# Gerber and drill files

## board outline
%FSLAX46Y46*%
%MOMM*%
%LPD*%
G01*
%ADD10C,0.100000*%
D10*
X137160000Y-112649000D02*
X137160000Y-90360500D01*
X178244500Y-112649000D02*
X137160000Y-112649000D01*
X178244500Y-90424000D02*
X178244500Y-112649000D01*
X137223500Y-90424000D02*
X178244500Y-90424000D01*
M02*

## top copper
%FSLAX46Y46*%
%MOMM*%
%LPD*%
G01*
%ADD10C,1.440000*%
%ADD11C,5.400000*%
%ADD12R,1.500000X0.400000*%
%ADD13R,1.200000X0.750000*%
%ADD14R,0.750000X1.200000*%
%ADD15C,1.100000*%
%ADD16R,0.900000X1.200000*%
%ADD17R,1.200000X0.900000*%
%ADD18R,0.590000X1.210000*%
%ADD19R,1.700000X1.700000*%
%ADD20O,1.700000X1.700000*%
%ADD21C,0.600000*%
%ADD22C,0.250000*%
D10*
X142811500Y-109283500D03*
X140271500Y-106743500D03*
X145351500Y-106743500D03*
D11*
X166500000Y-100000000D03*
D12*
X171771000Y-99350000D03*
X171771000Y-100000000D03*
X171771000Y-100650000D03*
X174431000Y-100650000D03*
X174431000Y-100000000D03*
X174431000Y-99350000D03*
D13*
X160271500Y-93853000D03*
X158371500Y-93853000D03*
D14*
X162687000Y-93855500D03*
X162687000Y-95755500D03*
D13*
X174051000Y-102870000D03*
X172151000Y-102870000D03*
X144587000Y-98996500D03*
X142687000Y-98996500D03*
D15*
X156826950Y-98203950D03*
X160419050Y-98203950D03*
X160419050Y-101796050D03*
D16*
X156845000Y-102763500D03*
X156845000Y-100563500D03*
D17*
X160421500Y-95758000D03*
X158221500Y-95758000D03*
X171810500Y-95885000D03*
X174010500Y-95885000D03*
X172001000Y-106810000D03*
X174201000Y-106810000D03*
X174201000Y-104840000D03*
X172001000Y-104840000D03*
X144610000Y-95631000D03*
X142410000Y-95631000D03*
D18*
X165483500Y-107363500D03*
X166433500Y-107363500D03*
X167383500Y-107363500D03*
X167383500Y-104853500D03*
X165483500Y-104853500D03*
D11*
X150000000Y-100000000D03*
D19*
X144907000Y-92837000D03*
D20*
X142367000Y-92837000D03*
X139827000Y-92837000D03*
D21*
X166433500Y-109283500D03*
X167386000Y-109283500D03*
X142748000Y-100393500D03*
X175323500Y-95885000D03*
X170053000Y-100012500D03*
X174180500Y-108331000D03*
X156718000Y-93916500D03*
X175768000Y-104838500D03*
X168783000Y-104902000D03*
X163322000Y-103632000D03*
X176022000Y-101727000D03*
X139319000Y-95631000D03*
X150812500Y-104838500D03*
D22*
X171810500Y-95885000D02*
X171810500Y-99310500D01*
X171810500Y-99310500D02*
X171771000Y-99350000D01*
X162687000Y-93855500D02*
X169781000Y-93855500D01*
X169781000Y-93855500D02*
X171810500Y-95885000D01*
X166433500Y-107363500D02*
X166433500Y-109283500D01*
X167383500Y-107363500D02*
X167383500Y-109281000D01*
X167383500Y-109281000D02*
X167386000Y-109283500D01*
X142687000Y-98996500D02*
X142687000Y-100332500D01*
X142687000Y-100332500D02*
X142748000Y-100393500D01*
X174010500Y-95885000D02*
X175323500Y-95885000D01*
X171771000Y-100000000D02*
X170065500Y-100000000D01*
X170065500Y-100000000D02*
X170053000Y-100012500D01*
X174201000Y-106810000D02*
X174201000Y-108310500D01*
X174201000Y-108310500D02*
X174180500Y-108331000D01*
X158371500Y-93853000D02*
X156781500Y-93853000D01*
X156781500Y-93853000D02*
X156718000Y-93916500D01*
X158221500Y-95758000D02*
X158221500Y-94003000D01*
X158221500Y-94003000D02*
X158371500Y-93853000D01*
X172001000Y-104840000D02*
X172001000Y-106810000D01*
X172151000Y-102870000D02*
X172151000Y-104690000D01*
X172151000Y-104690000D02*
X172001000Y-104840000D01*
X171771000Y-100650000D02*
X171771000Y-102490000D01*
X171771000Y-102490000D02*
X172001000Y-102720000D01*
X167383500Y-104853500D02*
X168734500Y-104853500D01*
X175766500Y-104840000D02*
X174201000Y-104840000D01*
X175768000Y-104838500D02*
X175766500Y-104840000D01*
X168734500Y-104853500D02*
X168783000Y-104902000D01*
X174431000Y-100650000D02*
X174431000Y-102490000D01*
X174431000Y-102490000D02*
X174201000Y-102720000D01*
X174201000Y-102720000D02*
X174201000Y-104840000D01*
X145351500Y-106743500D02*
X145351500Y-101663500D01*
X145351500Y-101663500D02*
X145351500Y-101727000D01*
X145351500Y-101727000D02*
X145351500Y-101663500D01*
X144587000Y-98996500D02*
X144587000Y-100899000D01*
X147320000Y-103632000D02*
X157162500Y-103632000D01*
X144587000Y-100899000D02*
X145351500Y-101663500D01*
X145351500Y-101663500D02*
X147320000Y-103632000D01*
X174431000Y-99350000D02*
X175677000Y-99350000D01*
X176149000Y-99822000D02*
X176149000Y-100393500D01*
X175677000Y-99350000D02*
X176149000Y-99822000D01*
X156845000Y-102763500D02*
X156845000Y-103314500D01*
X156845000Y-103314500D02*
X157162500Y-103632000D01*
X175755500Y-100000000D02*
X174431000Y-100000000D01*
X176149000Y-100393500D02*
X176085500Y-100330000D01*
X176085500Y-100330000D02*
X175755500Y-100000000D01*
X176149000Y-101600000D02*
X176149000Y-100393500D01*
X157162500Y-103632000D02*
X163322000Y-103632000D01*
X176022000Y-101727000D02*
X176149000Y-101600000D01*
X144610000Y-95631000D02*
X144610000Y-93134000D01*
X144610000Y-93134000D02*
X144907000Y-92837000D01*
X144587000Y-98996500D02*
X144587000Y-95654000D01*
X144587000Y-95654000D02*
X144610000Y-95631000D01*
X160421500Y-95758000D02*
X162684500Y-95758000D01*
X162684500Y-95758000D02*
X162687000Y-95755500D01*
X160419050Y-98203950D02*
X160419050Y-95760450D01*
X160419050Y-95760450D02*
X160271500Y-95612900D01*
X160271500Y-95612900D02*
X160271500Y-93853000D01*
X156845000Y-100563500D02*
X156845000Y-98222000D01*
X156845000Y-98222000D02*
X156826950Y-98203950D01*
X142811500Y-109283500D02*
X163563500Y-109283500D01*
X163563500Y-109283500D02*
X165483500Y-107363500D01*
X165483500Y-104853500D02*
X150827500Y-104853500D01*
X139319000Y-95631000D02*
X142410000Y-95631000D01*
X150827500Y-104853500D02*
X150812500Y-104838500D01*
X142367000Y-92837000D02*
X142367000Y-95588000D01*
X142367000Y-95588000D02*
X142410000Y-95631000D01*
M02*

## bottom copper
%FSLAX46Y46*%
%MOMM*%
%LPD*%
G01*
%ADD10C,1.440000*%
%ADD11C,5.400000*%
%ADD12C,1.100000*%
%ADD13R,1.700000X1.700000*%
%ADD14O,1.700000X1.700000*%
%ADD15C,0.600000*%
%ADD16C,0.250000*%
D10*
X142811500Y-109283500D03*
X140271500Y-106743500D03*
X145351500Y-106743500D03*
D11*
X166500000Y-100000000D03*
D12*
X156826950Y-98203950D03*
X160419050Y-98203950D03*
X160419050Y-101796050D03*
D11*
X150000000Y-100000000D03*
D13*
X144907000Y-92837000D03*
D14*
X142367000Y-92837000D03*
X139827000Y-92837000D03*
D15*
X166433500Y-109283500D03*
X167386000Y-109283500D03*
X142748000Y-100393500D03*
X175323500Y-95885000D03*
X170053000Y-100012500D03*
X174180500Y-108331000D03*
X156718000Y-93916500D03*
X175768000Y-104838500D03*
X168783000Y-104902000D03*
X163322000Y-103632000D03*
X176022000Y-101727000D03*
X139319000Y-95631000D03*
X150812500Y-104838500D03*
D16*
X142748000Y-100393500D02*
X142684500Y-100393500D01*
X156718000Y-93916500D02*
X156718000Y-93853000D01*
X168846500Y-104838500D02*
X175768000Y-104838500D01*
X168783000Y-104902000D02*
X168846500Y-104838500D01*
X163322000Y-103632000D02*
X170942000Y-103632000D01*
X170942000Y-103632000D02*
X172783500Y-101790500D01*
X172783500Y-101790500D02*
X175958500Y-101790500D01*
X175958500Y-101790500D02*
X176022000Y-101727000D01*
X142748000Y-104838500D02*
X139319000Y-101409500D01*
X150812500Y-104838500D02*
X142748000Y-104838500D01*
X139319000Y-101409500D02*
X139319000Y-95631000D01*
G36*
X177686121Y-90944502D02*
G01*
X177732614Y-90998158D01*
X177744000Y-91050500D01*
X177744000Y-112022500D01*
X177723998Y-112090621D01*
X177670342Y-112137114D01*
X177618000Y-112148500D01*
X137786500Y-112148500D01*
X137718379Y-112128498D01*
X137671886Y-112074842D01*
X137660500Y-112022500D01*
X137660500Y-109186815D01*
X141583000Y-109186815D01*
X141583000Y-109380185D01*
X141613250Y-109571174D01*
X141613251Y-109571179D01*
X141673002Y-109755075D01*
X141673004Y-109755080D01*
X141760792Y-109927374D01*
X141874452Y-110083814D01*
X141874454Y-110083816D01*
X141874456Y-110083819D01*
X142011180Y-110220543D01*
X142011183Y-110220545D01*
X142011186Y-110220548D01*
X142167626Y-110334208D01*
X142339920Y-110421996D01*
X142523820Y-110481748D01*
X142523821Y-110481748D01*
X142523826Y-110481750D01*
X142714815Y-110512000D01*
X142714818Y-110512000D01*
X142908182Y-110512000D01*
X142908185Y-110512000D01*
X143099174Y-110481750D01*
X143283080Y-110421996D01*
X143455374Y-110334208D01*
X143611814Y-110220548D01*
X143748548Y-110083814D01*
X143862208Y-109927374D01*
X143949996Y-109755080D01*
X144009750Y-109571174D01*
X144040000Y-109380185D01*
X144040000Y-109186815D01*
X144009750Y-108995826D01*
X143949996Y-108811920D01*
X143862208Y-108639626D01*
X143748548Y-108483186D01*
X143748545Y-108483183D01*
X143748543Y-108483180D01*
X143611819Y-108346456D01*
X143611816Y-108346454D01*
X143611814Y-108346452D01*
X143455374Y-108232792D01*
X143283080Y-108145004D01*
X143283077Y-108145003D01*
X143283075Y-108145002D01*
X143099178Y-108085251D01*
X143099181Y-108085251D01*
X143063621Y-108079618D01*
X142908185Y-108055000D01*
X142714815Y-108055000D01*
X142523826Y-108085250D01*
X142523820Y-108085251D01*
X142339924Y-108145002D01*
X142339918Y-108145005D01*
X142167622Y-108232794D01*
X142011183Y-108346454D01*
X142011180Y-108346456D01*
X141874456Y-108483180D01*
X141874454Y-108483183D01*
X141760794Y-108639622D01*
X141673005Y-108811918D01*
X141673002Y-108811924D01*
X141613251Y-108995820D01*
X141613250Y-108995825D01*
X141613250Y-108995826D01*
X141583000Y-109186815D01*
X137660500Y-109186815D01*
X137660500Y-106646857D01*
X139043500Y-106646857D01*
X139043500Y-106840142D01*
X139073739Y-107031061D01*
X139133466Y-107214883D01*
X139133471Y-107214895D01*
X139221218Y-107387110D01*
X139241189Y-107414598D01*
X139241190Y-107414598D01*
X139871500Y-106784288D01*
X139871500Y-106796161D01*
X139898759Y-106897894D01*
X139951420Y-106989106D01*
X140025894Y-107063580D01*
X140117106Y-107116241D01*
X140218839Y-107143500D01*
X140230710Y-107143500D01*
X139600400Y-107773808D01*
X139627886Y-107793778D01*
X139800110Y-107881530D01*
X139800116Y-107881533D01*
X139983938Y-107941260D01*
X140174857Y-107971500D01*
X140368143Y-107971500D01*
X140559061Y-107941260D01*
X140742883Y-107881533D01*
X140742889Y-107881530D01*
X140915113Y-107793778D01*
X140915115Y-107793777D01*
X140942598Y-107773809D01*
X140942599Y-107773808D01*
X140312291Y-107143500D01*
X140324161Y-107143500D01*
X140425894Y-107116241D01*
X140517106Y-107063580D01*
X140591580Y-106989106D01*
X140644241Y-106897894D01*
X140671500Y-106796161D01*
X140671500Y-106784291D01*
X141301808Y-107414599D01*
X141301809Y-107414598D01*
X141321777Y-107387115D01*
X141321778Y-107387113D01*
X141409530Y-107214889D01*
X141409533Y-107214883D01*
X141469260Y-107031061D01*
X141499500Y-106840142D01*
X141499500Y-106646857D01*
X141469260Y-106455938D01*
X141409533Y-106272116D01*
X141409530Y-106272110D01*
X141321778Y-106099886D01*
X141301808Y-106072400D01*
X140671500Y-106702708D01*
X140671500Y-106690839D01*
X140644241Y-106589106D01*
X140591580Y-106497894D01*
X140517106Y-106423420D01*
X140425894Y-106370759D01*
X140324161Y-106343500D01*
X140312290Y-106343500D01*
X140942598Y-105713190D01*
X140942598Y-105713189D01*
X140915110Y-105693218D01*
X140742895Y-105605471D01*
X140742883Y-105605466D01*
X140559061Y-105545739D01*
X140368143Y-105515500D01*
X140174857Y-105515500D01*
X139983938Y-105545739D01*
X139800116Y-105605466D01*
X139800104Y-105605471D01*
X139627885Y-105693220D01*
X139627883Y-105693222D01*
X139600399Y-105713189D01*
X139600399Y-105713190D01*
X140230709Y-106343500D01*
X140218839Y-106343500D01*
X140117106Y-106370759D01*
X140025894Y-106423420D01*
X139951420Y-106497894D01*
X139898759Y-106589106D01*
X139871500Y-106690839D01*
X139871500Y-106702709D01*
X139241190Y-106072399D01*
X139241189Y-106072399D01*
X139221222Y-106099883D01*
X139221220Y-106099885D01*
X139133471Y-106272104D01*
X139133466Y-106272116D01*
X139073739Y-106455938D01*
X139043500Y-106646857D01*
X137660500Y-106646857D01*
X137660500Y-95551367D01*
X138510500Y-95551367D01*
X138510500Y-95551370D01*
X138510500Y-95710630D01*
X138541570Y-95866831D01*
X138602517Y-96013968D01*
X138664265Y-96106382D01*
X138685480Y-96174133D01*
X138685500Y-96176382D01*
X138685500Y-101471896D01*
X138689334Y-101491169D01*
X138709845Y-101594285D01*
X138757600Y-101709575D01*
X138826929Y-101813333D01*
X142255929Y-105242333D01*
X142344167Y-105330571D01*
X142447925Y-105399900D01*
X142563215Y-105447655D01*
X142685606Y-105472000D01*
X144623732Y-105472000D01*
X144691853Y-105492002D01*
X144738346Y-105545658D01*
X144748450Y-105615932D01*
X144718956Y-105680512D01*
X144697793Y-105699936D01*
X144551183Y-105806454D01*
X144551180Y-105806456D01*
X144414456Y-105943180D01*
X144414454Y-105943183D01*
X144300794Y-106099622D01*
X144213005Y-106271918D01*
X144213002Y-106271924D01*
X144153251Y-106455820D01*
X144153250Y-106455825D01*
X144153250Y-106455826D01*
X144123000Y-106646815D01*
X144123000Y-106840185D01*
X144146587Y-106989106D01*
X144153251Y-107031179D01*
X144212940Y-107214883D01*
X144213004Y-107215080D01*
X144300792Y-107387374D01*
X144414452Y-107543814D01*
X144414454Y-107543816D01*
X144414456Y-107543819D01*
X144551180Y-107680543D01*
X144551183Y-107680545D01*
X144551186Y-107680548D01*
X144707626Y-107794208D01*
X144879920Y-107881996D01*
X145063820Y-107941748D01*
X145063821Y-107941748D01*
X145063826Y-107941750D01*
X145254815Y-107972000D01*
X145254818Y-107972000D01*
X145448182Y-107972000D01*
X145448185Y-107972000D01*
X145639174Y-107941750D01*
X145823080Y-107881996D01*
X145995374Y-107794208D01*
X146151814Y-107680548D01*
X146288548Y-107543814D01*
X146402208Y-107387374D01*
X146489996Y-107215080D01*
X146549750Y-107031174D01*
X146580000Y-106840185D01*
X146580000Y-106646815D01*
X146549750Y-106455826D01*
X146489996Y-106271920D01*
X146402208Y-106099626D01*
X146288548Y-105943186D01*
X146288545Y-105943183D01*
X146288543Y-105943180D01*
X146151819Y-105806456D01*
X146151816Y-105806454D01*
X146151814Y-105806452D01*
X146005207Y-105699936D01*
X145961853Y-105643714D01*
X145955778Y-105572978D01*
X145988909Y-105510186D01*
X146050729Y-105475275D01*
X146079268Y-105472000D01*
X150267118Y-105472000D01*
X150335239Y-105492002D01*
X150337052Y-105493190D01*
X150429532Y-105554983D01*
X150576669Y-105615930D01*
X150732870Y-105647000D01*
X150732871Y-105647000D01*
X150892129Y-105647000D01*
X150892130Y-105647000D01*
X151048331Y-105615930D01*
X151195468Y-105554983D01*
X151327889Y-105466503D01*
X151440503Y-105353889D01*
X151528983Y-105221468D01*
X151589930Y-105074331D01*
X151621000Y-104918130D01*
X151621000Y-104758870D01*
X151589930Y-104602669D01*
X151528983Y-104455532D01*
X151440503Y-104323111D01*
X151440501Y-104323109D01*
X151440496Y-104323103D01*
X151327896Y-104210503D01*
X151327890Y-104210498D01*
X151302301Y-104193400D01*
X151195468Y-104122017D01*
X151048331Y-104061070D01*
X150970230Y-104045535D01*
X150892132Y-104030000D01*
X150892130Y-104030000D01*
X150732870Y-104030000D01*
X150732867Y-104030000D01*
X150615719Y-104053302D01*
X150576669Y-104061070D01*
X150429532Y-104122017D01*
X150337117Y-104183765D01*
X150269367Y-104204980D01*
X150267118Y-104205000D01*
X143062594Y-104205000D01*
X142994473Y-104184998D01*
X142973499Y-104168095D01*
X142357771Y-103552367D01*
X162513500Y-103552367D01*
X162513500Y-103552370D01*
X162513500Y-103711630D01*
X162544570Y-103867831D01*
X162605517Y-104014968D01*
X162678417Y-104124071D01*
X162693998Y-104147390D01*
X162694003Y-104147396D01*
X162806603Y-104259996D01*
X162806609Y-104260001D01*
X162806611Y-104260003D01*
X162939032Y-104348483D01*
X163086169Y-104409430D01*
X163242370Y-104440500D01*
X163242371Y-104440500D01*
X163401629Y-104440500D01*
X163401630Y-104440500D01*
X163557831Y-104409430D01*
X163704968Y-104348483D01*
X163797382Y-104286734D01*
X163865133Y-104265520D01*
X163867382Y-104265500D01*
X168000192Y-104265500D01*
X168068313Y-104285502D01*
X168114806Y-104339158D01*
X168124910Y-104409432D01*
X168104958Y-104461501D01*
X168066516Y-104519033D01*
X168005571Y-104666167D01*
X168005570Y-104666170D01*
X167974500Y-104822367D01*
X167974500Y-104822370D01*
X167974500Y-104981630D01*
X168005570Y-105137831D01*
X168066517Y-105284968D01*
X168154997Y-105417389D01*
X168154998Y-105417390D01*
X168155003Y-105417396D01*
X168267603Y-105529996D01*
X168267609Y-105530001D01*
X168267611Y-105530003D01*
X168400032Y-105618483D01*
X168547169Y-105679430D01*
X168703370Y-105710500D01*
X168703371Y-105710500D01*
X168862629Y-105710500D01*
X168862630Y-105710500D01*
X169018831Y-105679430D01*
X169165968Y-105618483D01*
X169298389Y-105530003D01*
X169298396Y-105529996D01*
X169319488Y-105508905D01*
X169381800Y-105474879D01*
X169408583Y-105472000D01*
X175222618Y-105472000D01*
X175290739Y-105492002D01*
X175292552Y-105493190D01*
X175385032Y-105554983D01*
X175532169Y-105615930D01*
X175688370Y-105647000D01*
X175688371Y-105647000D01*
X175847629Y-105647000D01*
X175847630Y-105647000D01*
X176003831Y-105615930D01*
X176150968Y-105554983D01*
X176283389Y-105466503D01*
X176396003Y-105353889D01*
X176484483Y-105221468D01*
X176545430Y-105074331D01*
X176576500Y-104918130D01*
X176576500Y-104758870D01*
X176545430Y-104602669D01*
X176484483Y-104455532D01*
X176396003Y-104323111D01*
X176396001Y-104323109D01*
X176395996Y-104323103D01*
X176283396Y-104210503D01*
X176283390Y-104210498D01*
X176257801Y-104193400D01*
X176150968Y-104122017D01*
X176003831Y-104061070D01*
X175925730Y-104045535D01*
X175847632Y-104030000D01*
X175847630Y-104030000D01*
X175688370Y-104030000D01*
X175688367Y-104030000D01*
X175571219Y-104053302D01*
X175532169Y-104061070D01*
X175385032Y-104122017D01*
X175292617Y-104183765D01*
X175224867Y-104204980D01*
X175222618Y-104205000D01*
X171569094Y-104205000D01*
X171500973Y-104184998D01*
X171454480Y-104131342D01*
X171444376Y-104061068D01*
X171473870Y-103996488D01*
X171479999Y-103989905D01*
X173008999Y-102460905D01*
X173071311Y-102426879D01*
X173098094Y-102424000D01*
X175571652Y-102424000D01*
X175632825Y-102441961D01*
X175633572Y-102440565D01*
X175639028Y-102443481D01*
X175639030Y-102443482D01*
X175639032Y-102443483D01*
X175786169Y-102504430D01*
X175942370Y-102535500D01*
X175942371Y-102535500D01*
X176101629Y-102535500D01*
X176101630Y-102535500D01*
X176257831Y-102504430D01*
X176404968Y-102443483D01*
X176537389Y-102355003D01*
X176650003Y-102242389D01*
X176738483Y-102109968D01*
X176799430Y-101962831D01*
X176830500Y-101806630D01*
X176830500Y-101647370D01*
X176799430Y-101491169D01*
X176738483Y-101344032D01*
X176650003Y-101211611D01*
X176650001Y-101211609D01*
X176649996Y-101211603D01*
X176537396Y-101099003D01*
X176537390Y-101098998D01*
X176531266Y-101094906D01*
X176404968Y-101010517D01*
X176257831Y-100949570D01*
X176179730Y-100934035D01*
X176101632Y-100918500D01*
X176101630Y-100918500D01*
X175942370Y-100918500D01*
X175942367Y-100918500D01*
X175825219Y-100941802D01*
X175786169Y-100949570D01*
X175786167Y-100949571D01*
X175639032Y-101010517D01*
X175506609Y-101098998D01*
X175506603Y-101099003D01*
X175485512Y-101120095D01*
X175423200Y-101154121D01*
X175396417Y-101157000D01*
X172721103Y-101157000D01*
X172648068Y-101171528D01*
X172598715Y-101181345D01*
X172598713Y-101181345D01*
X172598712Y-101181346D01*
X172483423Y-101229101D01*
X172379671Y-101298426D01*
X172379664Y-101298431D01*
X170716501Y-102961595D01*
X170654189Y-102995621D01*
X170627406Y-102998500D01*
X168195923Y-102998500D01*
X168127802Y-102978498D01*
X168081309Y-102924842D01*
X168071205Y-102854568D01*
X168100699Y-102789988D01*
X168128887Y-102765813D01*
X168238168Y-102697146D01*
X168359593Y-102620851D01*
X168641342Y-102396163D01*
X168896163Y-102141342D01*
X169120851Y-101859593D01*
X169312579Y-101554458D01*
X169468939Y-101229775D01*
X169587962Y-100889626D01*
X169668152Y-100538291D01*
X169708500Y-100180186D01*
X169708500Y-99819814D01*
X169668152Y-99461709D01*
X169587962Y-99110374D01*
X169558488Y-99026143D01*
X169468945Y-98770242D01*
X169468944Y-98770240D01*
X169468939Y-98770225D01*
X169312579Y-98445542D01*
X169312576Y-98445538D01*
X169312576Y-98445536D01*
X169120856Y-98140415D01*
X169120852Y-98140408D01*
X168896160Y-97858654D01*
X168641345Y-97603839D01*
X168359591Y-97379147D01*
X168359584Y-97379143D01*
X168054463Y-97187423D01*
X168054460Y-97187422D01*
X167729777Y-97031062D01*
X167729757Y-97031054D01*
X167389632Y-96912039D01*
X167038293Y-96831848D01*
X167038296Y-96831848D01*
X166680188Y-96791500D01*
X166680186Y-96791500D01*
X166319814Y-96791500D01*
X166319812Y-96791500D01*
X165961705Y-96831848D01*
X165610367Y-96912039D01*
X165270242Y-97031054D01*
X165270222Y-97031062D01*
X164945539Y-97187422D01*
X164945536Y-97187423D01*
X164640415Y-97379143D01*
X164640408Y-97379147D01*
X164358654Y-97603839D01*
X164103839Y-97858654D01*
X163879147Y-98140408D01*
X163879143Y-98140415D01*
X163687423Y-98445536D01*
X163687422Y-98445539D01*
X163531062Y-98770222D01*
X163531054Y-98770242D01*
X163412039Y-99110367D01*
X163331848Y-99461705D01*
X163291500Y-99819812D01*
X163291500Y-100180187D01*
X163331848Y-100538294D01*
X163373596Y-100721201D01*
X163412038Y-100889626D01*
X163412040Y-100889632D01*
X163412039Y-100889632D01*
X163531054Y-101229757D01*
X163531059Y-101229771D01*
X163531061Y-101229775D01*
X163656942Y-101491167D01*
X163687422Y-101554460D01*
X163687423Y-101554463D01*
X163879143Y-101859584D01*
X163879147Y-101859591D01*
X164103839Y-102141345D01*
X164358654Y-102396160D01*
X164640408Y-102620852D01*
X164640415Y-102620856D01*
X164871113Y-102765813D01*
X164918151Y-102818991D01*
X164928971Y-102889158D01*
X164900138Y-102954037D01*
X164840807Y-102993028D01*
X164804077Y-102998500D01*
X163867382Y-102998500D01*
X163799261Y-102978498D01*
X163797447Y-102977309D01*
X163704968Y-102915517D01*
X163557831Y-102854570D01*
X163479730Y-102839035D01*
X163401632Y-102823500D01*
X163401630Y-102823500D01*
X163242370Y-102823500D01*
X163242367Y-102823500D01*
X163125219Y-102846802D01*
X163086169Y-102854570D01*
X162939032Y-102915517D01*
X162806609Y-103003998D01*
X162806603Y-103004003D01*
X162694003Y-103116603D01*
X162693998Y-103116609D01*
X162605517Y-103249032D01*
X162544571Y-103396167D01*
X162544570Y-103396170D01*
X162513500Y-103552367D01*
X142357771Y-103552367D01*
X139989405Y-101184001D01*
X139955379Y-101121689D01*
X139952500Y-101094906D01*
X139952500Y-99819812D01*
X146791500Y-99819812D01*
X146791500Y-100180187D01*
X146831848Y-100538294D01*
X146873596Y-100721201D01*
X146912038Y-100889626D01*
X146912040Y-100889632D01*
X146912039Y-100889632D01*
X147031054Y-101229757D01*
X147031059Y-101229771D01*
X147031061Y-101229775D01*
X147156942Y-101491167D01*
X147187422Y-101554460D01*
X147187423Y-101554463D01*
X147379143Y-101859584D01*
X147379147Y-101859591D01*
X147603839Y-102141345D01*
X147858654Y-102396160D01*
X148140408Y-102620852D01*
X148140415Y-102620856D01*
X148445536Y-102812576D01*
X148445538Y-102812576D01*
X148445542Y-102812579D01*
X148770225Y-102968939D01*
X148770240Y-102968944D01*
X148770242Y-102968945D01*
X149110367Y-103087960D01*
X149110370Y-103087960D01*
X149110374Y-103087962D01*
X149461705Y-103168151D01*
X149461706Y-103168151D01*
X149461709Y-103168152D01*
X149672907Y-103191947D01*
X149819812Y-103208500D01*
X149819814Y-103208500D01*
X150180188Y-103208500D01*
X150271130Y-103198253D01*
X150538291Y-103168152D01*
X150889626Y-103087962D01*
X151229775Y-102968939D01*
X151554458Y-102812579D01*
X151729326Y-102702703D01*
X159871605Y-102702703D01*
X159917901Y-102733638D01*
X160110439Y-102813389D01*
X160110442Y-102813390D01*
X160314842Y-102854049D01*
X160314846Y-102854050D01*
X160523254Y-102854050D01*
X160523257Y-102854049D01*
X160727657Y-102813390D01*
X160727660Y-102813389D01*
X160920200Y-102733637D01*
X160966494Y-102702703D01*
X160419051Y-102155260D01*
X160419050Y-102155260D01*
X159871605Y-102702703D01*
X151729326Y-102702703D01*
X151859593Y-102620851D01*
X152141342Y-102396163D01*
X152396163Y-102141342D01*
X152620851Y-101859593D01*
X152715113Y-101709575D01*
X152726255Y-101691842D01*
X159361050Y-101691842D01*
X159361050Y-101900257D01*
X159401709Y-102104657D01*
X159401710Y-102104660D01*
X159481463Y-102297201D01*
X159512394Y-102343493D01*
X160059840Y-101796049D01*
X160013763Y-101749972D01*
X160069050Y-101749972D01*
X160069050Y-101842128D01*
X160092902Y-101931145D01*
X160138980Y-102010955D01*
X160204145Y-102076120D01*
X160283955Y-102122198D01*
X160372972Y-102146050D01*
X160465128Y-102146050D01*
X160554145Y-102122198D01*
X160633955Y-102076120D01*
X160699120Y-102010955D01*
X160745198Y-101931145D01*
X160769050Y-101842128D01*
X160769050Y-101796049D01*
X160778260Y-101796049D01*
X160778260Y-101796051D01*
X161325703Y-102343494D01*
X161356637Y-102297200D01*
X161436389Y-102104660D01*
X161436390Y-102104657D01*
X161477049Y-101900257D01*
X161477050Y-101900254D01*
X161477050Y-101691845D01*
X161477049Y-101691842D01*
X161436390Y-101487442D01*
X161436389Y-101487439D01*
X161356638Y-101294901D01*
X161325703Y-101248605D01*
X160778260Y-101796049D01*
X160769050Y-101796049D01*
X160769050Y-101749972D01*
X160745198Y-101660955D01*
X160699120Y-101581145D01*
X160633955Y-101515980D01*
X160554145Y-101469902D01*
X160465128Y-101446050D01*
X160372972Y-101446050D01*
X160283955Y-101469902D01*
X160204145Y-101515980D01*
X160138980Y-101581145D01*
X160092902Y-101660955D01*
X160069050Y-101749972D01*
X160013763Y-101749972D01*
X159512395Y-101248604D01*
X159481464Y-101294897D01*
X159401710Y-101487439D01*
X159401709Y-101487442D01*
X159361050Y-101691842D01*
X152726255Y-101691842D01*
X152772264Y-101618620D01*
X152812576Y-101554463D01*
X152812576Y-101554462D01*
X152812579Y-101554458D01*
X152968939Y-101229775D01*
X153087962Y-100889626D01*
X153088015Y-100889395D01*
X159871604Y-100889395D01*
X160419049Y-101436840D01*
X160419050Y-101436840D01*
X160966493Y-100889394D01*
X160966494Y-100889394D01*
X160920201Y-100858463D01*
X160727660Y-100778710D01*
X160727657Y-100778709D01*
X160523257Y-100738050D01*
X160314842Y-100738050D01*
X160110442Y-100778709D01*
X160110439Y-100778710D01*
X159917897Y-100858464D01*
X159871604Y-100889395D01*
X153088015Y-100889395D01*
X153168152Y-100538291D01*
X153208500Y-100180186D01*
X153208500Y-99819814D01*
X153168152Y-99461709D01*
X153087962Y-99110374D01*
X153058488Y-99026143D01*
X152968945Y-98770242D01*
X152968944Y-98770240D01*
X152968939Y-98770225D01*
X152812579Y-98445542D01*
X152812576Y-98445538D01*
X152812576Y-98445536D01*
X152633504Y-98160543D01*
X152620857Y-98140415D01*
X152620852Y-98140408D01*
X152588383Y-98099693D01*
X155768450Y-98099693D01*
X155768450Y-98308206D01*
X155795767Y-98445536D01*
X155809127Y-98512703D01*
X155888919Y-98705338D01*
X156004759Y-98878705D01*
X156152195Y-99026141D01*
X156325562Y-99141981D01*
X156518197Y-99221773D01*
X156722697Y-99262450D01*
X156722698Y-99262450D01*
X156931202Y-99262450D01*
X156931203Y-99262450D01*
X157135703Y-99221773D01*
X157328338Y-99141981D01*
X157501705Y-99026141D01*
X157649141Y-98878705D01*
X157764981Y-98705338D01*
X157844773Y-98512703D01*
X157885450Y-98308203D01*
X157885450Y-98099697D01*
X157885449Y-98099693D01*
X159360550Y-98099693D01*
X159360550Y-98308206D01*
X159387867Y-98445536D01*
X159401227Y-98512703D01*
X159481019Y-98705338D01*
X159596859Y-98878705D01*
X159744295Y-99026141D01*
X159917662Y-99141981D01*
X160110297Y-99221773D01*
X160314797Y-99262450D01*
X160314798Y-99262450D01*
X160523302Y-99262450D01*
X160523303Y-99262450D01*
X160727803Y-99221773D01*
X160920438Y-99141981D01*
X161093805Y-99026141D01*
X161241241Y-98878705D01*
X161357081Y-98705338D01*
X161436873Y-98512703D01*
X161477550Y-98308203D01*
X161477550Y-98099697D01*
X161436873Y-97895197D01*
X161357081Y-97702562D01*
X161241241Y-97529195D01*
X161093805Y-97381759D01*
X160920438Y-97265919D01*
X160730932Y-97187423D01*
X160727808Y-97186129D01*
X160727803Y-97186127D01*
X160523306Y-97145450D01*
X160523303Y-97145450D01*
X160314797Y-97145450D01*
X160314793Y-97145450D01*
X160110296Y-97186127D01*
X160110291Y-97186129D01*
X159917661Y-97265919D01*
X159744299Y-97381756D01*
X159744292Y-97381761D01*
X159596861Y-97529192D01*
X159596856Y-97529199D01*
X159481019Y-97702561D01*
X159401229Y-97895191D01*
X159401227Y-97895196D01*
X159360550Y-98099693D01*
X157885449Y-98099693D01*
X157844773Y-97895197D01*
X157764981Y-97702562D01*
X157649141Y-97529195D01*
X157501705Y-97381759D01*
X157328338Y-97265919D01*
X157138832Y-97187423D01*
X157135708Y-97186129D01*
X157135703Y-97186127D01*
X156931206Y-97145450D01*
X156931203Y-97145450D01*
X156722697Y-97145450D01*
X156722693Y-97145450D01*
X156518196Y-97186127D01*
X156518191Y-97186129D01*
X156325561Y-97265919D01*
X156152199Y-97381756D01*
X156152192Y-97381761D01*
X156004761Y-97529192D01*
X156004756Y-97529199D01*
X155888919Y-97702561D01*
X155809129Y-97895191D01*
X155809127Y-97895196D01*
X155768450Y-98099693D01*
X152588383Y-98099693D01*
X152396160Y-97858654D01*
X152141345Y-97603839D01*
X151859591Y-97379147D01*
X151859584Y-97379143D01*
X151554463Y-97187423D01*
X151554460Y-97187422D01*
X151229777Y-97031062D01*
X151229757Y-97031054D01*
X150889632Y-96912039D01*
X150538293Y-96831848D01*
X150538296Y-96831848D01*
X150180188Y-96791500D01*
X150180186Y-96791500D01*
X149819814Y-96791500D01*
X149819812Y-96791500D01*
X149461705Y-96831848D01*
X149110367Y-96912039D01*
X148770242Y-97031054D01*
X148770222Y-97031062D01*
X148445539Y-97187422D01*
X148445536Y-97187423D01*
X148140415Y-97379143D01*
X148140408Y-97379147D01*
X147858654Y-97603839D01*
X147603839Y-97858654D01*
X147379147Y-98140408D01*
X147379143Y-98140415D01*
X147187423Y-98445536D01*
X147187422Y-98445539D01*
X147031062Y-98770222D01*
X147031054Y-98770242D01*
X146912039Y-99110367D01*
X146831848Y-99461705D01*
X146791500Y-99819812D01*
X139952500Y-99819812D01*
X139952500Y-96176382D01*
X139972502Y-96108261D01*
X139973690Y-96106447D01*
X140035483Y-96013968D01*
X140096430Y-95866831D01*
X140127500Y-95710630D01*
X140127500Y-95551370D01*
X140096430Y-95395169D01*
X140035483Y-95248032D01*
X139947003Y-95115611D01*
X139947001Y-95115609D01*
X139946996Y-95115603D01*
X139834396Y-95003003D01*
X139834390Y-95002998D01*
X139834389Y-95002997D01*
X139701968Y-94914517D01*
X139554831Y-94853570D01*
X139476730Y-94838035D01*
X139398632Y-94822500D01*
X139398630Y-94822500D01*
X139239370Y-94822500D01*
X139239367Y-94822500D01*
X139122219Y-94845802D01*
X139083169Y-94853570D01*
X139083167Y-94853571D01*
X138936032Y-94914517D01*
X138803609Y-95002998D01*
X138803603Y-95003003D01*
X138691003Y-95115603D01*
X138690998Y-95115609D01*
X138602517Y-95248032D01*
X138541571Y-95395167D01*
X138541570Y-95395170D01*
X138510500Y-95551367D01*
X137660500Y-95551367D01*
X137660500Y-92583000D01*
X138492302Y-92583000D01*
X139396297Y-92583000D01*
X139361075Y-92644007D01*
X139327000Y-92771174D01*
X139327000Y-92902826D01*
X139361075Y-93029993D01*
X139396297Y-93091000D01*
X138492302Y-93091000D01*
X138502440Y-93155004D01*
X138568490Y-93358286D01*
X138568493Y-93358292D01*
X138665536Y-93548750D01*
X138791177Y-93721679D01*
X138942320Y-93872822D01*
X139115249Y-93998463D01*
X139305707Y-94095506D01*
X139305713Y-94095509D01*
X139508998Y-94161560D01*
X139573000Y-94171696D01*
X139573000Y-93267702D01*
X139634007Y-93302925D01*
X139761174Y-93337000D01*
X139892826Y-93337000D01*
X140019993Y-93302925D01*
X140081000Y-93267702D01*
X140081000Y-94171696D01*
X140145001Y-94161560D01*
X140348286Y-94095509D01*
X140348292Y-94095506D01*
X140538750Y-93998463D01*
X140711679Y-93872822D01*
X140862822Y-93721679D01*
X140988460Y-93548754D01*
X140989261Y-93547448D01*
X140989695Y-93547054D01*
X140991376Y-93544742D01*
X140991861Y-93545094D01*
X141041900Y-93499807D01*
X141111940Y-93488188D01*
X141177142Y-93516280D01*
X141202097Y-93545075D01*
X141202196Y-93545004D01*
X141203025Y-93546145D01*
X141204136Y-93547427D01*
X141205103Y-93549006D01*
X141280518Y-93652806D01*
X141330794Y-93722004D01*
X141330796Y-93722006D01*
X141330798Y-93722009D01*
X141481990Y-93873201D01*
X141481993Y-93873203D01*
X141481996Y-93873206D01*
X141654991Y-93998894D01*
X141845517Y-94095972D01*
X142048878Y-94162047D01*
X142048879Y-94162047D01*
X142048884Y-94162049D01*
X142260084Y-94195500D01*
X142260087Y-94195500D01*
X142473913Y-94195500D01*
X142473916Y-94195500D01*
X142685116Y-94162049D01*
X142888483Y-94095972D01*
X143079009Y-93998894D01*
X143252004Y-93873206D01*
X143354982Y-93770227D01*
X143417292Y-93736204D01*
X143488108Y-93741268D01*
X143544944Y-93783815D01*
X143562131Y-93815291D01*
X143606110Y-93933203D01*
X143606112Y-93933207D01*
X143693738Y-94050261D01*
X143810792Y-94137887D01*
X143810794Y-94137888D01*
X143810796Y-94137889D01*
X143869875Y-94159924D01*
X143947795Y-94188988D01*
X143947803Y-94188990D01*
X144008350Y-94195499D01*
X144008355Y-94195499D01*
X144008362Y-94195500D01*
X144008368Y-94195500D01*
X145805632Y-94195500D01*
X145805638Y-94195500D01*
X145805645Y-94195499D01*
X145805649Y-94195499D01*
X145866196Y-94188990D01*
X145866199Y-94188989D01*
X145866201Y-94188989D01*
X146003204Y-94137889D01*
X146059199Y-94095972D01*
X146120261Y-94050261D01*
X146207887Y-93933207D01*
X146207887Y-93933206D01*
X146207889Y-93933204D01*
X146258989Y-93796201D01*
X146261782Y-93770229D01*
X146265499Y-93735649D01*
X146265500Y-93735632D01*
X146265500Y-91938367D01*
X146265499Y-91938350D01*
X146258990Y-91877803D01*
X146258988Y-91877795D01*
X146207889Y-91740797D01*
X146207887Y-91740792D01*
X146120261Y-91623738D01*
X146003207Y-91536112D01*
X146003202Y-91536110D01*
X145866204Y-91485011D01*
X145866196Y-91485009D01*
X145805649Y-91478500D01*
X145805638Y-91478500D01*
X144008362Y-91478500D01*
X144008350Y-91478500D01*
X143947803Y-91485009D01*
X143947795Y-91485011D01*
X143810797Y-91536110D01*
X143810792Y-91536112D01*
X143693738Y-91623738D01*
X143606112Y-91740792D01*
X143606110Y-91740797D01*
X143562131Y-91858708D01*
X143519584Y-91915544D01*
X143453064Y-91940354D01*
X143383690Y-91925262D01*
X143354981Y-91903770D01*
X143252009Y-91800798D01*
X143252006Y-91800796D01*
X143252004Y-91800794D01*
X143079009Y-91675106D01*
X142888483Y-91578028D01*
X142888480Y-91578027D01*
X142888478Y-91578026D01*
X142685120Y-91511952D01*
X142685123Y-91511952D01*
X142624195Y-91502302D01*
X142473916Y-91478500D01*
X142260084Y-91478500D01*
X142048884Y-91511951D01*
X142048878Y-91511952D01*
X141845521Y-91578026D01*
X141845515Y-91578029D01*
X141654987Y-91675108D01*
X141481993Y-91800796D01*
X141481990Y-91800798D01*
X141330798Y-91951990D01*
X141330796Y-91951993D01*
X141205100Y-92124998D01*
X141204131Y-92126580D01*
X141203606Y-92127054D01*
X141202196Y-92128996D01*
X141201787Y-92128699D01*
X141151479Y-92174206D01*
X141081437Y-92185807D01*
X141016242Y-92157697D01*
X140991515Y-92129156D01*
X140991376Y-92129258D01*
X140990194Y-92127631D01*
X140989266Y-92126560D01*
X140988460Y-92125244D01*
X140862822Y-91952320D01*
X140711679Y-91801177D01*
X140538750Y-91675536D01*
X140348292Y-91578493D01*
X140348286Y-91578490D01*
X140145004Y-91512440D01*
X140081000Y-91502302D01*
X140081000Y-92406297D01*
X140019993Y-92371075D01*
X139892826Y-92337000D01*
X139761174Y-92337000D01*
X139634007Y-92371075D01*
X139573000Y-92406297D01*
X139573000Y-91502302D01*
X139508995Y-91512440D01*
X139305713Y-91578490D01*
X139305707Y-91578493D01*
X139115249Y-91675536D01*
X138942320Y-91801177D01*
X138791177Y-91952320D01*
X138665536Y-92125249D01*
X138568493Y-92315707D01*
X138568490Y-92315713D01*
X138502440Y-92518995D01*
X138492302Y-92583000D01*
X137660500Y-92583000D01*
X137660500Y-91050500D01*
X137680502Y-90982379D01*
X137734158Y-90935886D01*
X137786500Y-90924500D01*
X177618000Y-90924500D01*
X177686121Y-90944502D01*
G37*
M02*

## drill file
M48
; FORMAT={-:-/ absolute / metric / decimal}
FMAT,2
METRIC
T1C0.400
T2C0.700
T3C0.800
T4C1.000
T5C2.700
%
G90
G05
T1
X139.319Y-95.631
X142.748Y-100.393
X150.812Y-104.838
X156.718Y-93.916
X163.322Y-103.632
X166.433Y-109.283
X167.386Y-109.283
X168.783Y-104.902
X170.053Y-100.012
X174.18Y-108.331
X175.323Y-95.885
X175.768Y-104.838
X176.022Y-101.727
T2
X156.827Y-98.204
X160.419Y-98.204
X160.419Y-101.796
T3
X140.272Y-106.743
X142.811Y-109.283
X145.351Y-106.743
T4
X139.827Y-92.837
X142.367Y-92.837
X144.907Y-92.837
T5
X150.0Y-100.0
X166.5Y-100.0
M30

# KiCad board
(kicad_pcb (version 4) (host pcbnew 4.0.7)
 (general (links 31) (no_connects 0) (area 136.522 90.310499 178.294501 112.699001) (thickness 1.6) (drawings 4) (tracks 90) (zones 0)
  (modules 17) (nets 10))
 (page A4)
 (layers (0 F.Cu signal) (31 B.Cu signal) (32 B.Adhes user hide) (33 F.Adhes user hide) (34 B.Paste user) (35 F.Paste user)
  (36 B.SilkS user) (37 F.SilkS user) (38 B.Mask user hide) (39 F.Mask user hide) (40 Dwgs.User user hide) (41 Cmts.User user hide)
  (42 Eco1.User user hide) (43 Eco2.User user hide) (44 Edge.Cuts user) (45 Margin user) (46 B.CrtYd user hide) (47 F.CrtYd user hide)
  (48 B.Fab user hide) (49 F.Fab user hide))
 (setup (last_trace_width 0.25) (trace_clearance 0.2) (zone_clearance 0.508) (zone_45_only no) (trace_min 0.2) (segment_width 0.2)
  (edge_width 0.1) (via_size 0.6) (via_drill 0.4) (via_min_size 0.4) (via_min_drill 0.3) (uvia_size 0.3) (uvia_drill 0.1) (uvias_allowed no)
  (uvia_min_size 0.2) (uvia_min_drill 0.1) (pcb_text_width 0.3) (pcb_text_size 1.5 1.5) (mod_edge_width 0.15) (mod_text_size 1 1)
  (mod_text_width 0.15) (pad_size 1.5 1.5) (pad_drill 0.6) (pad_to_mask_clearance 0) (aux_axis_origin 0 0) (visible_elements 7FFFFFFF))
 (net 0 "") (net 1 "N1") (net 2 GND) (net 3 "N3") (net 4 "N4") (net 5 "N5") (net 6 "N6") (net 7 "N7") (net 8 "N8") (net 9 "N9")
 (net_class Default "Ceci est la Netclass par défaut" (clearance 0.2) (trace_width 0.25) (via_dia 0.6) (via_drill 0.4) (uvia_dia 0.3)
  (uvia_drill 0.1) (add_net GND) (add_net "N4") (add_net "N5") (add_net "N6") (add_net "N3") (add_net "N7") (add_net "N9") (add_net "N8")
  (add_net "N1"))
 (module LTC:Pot (layer B.Cu) (at 145.3515 106.7435 180)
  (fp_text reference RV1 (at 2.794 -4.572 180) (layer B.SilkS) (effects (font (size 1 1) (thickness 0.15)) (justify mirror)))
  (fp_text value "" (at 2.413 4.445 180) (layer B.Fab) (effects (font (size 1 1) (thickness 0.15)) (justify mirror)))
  (pad 2 thru_hole circle (at 2.54 -2.54 180) (size 1.44 1.44) (drill 0.8) (layers *.Cu *.Mask) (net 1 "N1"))
  (pad 3 thru_hole circle (at 5.08 0 180) (size 1.44 1.44) (drill 0.8) (layers *.Cu *.Mask) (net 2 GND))
  (pad 1 thru_hole circle (at 0 0 180) (size 1.44 1.44) (drill 0.8) (layers *.Cu *.Mask) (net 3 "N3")))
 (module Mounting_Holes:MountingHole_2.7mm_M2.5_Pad (layer F.Cu) (at 166.5 100)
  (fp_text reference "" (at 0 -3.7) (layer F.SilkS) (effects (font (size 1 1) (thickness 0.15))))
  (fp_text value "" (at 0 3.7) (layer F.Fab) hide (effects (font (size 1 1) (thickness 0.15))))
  (pad 1 thru_hole circle (at 0 0) (size 5.4 5.4) (drill 2.7) (layers *.Cu *.Mask)))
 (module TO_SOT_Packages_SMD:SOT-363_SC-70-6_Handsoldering (layer F.Cu) (at 173.101 100)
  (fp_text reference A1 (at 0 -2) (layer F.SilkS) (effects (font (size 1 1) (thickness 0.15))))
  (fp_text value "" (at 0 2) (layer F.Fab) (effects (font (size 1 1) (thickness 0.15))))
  (pad 1 smd rect (at -1.33 -0.65) (size 1.5 0.4) (layers F.Cu F.Paste F.Mask) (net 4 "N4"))
  (pad 2 smd rect (at -1.33 0) (size 1.5 0.4) (layers F.Cu F.Paste F.Mask) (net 2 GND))
  (pad 3 smd rect (at -1.33 0.65) (size 1.5 0.4) (layers F.Cu F.Paste F.Mask) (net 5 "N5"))
  (pad 4 smd rect (at 1.33 0.65) (size 1.5 0.4) (layers F.Cu F.Paste F.Mask) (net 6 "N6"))
  (pad 5 smd rect (at 1.33 0) (size 1.5 0.4) (layers F.Cu F.Paste F.Mask) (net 3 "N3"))
  (pad 6 smd rect (at 1.33 -0.65) (size 1.5 0.4) (layers F.Cu F.Paste F.Mask) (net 3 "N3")))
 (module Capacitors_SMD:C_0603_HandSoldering (layer F.Cu) (at 159.3215 93.853 180)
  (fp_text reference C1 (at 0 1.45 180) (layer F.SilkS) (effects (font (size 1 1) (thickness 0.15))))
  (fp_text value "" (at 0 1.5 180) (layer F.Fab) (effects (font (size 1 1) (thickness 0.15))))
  (pad 1 smd rect (at -0.95 0 180) (size 1.2 0.75) (layers F.Cu F.Paste F.Mask) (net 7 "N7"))
  (pad 2 smd rect (at 0.95 0 180) (size 1.2 0.75) (layers F.Cu F.Paste F.Mask) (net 2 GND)))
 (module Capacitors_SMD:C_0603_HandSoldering (layer F.Cu) (at 162.687 94.8055 270)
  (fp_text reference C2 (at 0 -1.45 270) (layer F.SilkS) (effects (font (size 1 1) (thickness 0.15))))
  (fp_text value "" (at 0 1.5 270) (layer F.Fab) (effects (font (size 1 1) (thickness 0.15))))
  (pad 1 smd rect (at -0.95 0 270) (size 1.2 0.75) (layers F.Cu F.Paste F.Mask) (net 4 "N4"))
  (pad 2 smd rect (at 0.95 0 270) (size 1.2 0.75) (layers F.Cu F.Paste F.Mask) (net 7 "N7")))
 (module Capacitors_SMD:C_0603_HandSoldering (layer F.Cu) (at 173.101 102.87 180)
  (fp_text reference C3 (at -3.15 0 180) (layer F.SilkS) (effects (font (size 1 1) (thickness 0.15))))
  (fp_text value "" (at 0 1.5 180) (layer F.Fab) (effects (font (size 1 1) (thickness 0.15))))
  (pad 1 smd rect (at -0.95 0 180) (size 1.2 0.75) (layers F.Cu F.Paste F.Mask) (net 6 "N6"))
  (pad 2 smd rect (at 0.95 0 180) (size 1.2 0.75) (layers F.Cu F.Paste F.Mask) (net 5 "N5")))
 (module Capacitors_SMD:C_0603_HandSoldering (layer F.Cu) (at 143.637 98.9965 180)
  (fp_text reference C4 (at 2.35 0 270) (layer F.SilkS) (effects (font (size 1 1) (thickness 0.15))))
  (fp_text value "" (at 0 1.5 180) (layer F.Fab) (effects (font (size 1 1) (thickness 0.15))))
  (pad 1 smd rect (at -0.95 0 180) (size 1.2 0.75) (layers F.Cu F.Paste F.Mask) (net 3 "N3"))
  (pad 2 smd rect (at 0.95 0 180) (size 1.2 0.75) (layers F.Cu F.Paste F.Mask) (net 2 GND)))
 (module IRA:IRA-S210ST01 (layer B.Cu) (at 158.623 100)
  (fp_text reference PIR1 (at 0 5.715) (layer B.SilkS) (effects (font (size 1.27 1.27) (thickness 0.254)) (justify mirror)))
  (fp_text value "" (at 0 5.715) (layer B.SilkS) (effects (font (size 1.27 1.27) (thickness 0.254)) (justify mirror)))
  (pad 1 thru_hole circle (at -1.79605 -1.79605 270) (size 1.1 1.1) (drill 0.7) (layers *.Cu *.Mask B.SilkS) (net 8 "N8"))
  (pad 2 thru_hole circle (at 1.79605 -1.79605 270) (size 1.1 1.1) (drill 0.7) (layers *.Cu *.Mask B.SilkS) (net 7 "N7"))
  (pad 3 thru_hole circle (at 1.79605 1.79605 270) (size 1.1 1.1) (drill 0.7) (layers *.Cu *.Mask B.SilkS) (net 2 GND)))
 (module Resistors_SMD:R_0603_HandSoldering (layer F.Cu) (at 156.845 101.6635 90)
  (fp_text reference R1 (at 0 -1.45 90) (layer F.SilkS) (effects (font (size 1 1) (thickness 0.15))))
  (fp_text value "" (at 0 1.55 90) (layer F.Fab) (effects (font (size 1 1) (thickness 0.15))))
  (pad 1 smd rect (at -1.1 0 90) (size 1.2 0.9) (layers F.Cu F.Paste F.Mask) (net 3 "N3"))
  (pad 2 smd rect (at 1.1 0 90) (size 1.2 0.9) (layers F.Cu F.Paste F.Mask) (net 8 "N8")))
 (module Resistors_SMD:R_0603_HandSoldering (layer F.Cu) (at 159.3215 95.758 180)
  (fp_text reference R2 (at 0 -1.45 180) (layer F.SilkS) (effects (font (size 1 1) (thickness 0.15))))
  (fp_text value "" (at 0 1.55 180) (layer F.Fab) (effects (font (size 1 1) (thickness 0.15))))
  (pad 1 smd rect (at -1.1 0 180) (size 1.2 0.9) (layers F.Cu F.Paste F.Mask) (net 7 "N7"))
  (pad 2 smd rect (at 1.1 0 180) (size 1.2 0.9) (layers F.Cu F.Paste F.Mask) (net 2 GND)))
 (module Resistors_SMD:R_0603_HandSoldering (layer F.Cu) (at 172.9105 95.885)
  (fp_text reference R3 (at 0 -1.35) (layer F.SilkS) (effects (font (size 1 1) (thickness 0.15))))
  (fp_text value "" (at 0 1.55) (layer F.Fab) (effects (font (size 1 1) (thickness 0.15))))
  (pad 1 smd rect (at -1.1 0) (size 1.2 0.9) (layers F.Cu F.Paste F.Mask) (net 4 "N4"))
  (pad 2 smd rect (at 1.1 0) (size 1.2 0.9) (layers F.Cu F.Paste F.Mask) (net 2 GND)))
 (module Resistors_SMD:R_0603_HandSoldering (layer F.Cu) (at 173.101 106.81)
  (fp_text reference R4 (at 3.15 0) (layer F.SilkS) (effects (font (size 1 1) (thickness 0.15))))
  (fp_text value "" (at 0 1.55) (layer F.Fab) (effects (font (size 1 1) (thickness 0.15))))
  (pad 1 smd rect (at -1.1 0) (size 1.2 0.9) (layers F.Cu F.Paste F.Mask) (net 5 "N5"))
  (pad 2 smd rect (at 1.1 0) (size 1.2 0.9) (layers F.Cu F.Paste F.Mask) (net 2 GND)))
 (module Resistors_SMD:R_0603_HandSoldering (layer F.Cu) (at 173.101 104.84 180)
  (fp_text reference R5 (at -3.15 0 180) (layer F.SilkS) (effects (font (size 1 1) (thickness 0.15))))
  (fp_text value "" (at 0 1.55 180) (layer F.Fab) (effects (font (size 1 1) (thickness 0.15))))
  (pad 1 smd rect (at -1.1 0 180) (size 1.2 0.9) (layers F.Cu F.Paste F.Mask) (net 6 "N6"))
  (pad 2 smd rect (at 1.1 0 180) (size 1.2 0.9) (layers F.Cu F.Paste F.Mask) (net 5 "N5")))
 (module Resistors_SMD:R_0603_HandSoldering (layer F.Cu) (at 143.51 95.631 180)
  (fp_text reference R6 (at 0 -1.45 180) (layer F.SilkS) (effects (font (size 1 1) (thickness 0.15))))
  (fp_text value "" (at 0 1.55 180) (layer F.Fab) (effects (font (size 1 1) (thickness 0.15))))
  (pad 1 smd rect (at -1.1 0 180) (size 1.2 0.9) (layers F.Cu F.Paste F.Mask) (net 3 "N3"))
  (pad 2 smd rect (at 1.1 0 180) (size 1.2 0.9) (layers F.Cu F.Paste F.Mask) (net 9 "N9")))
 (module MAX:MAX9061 (layer F.Cu) (at 166.4335 106.1085 90)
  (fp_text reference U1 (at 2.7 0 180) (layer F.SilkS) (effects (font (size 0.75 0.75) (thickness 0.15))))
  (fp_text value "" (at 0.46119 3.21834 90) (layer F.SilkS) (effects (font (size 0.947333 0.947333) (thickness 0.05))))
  (pad 1 smd rect (at -1.255 -0.95 270) (size 1.21 0.59) (layers F.Cu F.Paste F.Mask) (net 1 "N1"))
  (pad 2 smd rect (at -1.255 0 270) (size 1.21 0.59) (layers F.Cu F.Paste F.Mask) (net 2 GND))
  (pad 3 smd rect (at -1.255 0.95 270) (size 1.21 0.59) (layers F.Cu F.Paste F.Mask) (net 2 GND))
  (pad 4 smd rect (at 1.255 0.95 90) (size 1.21 0.59) (layers F.Cu F.Paste F.Mask) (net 6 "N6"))
  (pad 5 smd rect (at 1.255 -0.95 90) (size 1.21 0.59) (layers F.Cu F.Paste F.Mask) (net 9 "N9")))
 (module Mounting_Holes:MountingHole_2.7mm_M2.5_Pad (layer F.Cu) (at 150 100)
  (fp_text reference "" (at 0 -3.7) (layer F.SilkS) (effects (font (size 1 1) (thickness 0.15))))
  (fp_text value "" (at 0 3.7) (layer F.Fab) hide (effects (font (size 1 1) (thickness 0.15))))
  (pad 1 thru_hole circle (at 0 0) (size 5.4 5.4) (drill 2.7) (layers *.Cu *.Mask)))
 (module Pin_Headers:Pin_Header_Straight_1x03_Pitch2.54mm (layer F.Cu) (at 144.907 92.837 270)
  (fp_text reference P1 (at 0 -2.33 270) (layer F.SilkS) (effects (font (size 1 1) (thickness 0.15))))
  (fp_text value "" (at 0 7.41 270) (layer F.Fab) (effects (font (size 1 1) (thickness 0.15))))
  (pad 1 thru_hole rect (at 0 0 270) (size 1.7 1.7) (drill 1) (layers *.Cu *.Mask) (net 3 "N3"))
  (pad 2 thru_hole oval (at 0 2.54 270) (size 1.7 1.7) (drill 1) (layers *.Cu *.Mask) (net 9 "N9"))
  (pad 3 thru_hole oval (at 0 5.08 270) (size 1.7 1.7) (drill 1) (layers *.Cu *.Mask) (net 2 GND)))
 (gr_line (start 137.16 112.649) (end 137.16 90.3605) (angle 90) (layer Edge.Cuts) (width 0.1))
 (gr_line (start 178.2445 112.649) (end 137.16 112.649) (angle 90) (layer Edge.Cuts) (width 0.1))
 (gr_line (start 178.2445 90.424) (end 178.2445 112.649) (angle 90) (layer Edge.Cuts) (width 0.1))
 (gr_line (start 137.2235 90.424) (end 178.2445 90.424) (angle 90) (layer Edge.Cuts) (width 0.1))
 (segment (start 171.8105 95.885) (end 171.8105 99.3105) (width 0.25) (layer F.Cu) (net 4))
 (segment (start 171.8105 99.3105) (end 171.771 99.35) (width 0.25) (layer F.Cu) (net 4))
 (segment (start 162.687 93.8555) (end 169.781 93.8555) (width 0.25) (layer F.Cu) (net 4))
 (segment (start 169.781 93.8555) (end 171.8105 95.885) (width 0.25) (layer F.Cu) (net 4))
 (segment (start 166.4335 107.3635) (end 166.4335 109.2835) (width 0.25) (layer F.Cu) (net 2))
 (via (at 166.4335 109.2835) (size 0.6) (drill 0.4) (layers F.Cu B.Cu) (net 2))
 (segment (start 167.3835 107.3635) (end 167.3835 109.281) (width 0.25) (layer F.Cu) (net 2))
 (via (at 167.386 109.2835) (size 0.6) (drill 0.4) (layers F.Cu B.Cu) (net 2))
 (segment (start 167.3835 109.281) (end 167.386 109.2835) (width 0.25) (layer F.Cu) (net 2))
 (segment (start 142.687 98.9965) (end 142.687 100.3325) (width 0.25) (layer F.Cu) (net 2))
 (segment (start 142.748 100.3935) (end 142.6845 100.3935) (width 0.25) (layer B.Cu) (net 2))
 (via (at 142.748 100.3935) (size 0.6) (drill 0.4) (layers F.Cu B.Cu) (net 2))
 (segment (start 142.687 100.3325) (end 142.748 100.3935) (width 0.25) (layer F.Cu) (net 2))
 (segment (start 174.0105 95.885) (end 175.3235 95.885) (width 0.25) (layer F.Cu) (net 2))
 (via (at 175.3235 95.885) (size 0.6) (drill 0.4) (layers F.Cu B.Cu) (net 2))
 (segment (start 171.771 100) (end 170.0655 100) (width 0.25) (layer F.Cu) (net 2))
 (via (at 170.053 100.0125) (size 0.6) (drill 0.4) (layers F.Cu B.Cu) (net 2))
 (segment (start 170.0655 100) (end 170.053 100.0125) (width 0.25) (layer F.Cu) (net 2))
 (segment (start 174.201 106.81) (end 174.201 108.3105) (width 0.25) (layer F.Cu) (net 2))
 (via (at 174.1805 108.331) (size 0.6) (drill 0.4) (layers F.Cu B.Cu) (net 2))
 (segment (start 174.201 108.3105) (end 174.1805 108.331) (width 0.25) (layer F.Cu) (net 2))
 (segment (start 158.3715 93.853) (end 156.7815 93.853) (width 0.25) (layer F.Cu) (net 2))
 (segment (start 156.718 93.9165) (end 156.718 93.853) (width 0.25) (layer B.Cu) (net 2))
 (via (at 156.718 93.9165) (size 0.6) (drill 0.4) (layers F.Cu B.Cu) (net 2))
 (segment (start 156.7815 93.853) (end 156.718 93.9165) (width 0.25) (layer F.Cu) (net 2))
 (segment (start 158.2215 95.758) (end 158.2215 94.003) (width 0.25) (layer F.Cu) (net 2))
 (segment (start 158.2215 94.003) (end 158.3715 93.853) (width 0.25) (layer F.Cu) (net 2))
 (segment (start 172.001 104.84) (end 172.001 106.81) (width 0.25) (layer F.Cu) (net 5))
 (segment (start 172.151 102.87) (end 172.151 104.69) (width 0.25) (layer F.Cu) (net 5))
 (segment (start 172.151 104.69) (end 172.001 104.84) (width 0.25) (layer F.Cu) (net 5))
 (segment (start 171.771 100.65) (end 171.771 102.49) (width 0.25) (layer F.Cu) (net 5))
 (segment (start 171.771 102.49) (end 172.001 102.72) (width 0.25) (layer F.Cu) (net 5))
 (segment (start 167.3835 104.8535) (end 168.7345 104.8535) (width 0.25) (layer F.Cu) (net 6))
 (segment (start 175.7665 104.84) (end 174.201 104.84) (width 0.25) (layer F.Cu) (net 6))
 (segment (start 175.768 104.8385) (end 175.7665 104.84) (width 0.25) (layer F.Cu) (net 6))
 (via (at 175.768 104.8385) (size 0.6) (drill 0.4) (layers F.Cu B.Cu) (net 6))
 (segment (start 168.8465 104.8385) (end 175.768 104.8385) (width 0.25) (layer B.Cu) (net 6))
 (segment (start 168.783 104.902) (end 168.8465 104.8385) (width 0.25) (layer B.Cu) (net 6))
 (via (at 168.783 104.902) (size 0.6) (drill 0.4) (layers F.Cu B.Cu) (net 6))
 (segment (start 168.7345 104.8535) (end 168.783 104.902) (width 0.25) (layer F.Cu) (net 6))
 (segment (start 174.431 100.65) (end 174.431 102.49) (width 0.25) (layer F.Cu) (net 6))
 (segment (start 174.431 102.49) (end 174.201 102.72) (width 0.25) (layer F.Cu) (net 6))
 (segment (start 174.201 102.72) (end 174.201 104.84) (width 0.25) (layer F.Cu) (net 6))
 (segment (start 145.3515 106.7435) (end 145.3515 101.6635) (width 0.25) (layer F.Cu) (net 3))
 (segment (start 145.3515 101.6635) (end 145.3515 101.727) (width 0.25) (layer F.Cu) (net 3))
 (segment (start 145.3515 101.727) (end 145.3515 101.6635) (width 0.25) (layer F.Cu) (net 3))
 (segment (start 144.587 98.9965) (end 144.587 100.899) (width 0.25) (layer F.Cu) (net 3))
 (segment (start 147.32 103.632) (end 157.1625 103.632) (width 0.25) (layer F.Cu) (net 3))
 (segment (start 144.587 100.899) (end 145.3515 101.6635) (width 0.25) (layer F.Cu) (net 3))
 (segment (start 145.3515 101.6635) (end 147.32 103.632) (width 0.25) (layer F.Cu) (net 3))
 (segment (start 174.431 99.35) (end 175.677 99.35) (width 0.25) (layer F.Cu) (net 3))
 (segment (start 176.149 99.822) (end 176.149 100.3935) (width 0.25) (layer F.Cu) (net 3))
 (segment (start 175.677 99.35) (end 176.149 99.822) (width 0.25) (layer F.Cu) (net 3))
 (segment (start 156.845 102.7635) (end 156.845 103.3145) (width 0.25) (layer F.Cu) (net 3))
 (segment (start 156.845 103.3145) (end 157.1625 103.632) (width 0.25) (layer F.Cu) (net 3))
 (segment (start 175.7555 100) (end 174.431 100) (width 0.25) (layer F.Cu) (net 3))
 (segment (start 176.149 100.3935) (end 176.0855 100.33) (width 0.25) (layer F.Cu) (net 3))
 (segment (start 176.0855 100.33) (end 175.7555 100) (width 0.25) (layer F.Cu) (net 3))
 (segment (start 176.149 101.6) (end 176.149 100.3935) (width 0.25) (layer F.Cu) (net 3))
 (segment (start 157.1625 103.632) (end 163.322 103.632) (width 0.25) (layer F.Cu) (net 3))
 (via (at 163.322 103.632) (size 0.6) (drill 0.4) (layers F.Cu B.Cu) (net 3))
 (segment (start 163.322 103.632) (end 170.942 103.632) (width 0.25) (layer B.Cu) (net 3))
 (segment (start 170.942 103.632) (end 172.7835 101.7905) (width 0.25) (layer B.Cu) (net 3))
 (segment (start 172.7835 101.7905) (end 175.9585 101.7905) (width 0.25) (layer B.Cu) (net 3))
 (segment (start 175.9585 101.7905) (end 176.022 101.727) (width 0.25) (layer B.Cu) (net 3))
 (via (at 176.022 101.727) (size 0.6) (drill 0.4) (layers F.Cu B.Cu) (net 3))
 (segment (start 176.022 101.727) (end 176.149 101.6) (width 0.25) (layer F.Cu) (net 3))
 (segment (start 144.61 95.631) (end 144.61 93.134) (width 0.25) (layer F.Cu) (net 3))
 (segment (start 144.61 93.134) (end 144.907 92.837) (width 0.25) (layer F.Cu) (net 3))
 (segment (start 144.587 98.9965) (end 144.587 95.654) (width 0.25) (layer F.Cu) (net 3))
 (segment (start 144.587 95.654) (end 144.61 95.631) (width 0.25) (layer F.Cu) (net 3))
 (segment (start 160.4215 95.758) (end 162.6845 95.758) (width 0.25) (layer F.Cu) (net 7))
 (segment (start 162.6845 95.758) (end 162.687 95.7555) (width 0.25) (layer F.Cu) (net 7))
 (segment (start 160.41905 98.20395) (end 160.41905 95.76045) (width 0.25) (layer F.Cu) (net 7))
 (segment (start 160.41905 95.76045) (end 160.2715 95.6129) (width 0.25) (layer F.Cu) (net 7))
 (segment (start 160.2715 95.6129) (end 160.2715 93.853) (width 0.25) (layer F.Cu) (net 7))
 (segment (start 156.845 100.5635) (end 156.845 98.222) (width 0.25) (layer F.Cu) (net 8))
 (segment (start 156.845 98.222) (end 156.82695 98.20395) (width 0.25) (layer F.Cu) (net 8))
 (segment (start 142.8115 109.2835) (end 163.5635 109.2835) (width 0.25) (layer F.Cu) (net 1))
 (segment (start 163.5635 109.2835) (end 165.4835 107.3635) (width 0.25) (layer F.Cu) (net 1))
 (segment (start 142.748 104.8385) (end 139.319 101.4095) (width 0.25) (layer B.Cu) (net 9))
 (segment (start 150.8125 104.8385) (end 142.748 104.8385) (width 0.25) (layer B.Cu) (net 9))
 (segment (start 165.4835 104.8535) (end 150.8275 104.8535) (width 0.25) (layer F.Cu) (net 9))
 (segment (start 139.319 95.631) (end 142.41 95.631) (width 0.25) (layer F.Cu) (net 9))
 (via (at 139.319 95.631) (size 0.6) (drill 0.4) (layers F.Cu B.Cu) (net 9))
 (segment (start 139.319 101.4095) (end 139.319 95.631) (width 0.25) (layer B.Cu) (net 9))
 (via (at 150.8125 104.8385) (size 0.6) (drill 0.4) (layers F.Cu B.Cu) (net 9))
 (segment (start 150.8275 104.8535) (end 150.8125 104.8385) (width 0.25) (layer F.Cu) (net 9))
 (segment (start 142.367 92.837) (end 142.367 95.588) (width 0.25) (layer F.Cu) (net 9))
 (segment (start 142.367 95.588) (end 142.41 95.631) (width 0.25) (layer F.Cu) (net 9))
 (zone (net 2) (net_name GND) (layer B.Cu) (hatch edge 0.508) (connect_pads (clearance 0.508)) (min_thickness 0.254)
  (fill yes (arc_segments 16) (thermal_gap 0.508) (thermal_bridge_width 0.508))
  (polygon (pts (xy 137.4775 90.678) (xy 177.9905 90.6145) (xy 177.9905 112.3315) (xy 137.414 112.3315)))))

